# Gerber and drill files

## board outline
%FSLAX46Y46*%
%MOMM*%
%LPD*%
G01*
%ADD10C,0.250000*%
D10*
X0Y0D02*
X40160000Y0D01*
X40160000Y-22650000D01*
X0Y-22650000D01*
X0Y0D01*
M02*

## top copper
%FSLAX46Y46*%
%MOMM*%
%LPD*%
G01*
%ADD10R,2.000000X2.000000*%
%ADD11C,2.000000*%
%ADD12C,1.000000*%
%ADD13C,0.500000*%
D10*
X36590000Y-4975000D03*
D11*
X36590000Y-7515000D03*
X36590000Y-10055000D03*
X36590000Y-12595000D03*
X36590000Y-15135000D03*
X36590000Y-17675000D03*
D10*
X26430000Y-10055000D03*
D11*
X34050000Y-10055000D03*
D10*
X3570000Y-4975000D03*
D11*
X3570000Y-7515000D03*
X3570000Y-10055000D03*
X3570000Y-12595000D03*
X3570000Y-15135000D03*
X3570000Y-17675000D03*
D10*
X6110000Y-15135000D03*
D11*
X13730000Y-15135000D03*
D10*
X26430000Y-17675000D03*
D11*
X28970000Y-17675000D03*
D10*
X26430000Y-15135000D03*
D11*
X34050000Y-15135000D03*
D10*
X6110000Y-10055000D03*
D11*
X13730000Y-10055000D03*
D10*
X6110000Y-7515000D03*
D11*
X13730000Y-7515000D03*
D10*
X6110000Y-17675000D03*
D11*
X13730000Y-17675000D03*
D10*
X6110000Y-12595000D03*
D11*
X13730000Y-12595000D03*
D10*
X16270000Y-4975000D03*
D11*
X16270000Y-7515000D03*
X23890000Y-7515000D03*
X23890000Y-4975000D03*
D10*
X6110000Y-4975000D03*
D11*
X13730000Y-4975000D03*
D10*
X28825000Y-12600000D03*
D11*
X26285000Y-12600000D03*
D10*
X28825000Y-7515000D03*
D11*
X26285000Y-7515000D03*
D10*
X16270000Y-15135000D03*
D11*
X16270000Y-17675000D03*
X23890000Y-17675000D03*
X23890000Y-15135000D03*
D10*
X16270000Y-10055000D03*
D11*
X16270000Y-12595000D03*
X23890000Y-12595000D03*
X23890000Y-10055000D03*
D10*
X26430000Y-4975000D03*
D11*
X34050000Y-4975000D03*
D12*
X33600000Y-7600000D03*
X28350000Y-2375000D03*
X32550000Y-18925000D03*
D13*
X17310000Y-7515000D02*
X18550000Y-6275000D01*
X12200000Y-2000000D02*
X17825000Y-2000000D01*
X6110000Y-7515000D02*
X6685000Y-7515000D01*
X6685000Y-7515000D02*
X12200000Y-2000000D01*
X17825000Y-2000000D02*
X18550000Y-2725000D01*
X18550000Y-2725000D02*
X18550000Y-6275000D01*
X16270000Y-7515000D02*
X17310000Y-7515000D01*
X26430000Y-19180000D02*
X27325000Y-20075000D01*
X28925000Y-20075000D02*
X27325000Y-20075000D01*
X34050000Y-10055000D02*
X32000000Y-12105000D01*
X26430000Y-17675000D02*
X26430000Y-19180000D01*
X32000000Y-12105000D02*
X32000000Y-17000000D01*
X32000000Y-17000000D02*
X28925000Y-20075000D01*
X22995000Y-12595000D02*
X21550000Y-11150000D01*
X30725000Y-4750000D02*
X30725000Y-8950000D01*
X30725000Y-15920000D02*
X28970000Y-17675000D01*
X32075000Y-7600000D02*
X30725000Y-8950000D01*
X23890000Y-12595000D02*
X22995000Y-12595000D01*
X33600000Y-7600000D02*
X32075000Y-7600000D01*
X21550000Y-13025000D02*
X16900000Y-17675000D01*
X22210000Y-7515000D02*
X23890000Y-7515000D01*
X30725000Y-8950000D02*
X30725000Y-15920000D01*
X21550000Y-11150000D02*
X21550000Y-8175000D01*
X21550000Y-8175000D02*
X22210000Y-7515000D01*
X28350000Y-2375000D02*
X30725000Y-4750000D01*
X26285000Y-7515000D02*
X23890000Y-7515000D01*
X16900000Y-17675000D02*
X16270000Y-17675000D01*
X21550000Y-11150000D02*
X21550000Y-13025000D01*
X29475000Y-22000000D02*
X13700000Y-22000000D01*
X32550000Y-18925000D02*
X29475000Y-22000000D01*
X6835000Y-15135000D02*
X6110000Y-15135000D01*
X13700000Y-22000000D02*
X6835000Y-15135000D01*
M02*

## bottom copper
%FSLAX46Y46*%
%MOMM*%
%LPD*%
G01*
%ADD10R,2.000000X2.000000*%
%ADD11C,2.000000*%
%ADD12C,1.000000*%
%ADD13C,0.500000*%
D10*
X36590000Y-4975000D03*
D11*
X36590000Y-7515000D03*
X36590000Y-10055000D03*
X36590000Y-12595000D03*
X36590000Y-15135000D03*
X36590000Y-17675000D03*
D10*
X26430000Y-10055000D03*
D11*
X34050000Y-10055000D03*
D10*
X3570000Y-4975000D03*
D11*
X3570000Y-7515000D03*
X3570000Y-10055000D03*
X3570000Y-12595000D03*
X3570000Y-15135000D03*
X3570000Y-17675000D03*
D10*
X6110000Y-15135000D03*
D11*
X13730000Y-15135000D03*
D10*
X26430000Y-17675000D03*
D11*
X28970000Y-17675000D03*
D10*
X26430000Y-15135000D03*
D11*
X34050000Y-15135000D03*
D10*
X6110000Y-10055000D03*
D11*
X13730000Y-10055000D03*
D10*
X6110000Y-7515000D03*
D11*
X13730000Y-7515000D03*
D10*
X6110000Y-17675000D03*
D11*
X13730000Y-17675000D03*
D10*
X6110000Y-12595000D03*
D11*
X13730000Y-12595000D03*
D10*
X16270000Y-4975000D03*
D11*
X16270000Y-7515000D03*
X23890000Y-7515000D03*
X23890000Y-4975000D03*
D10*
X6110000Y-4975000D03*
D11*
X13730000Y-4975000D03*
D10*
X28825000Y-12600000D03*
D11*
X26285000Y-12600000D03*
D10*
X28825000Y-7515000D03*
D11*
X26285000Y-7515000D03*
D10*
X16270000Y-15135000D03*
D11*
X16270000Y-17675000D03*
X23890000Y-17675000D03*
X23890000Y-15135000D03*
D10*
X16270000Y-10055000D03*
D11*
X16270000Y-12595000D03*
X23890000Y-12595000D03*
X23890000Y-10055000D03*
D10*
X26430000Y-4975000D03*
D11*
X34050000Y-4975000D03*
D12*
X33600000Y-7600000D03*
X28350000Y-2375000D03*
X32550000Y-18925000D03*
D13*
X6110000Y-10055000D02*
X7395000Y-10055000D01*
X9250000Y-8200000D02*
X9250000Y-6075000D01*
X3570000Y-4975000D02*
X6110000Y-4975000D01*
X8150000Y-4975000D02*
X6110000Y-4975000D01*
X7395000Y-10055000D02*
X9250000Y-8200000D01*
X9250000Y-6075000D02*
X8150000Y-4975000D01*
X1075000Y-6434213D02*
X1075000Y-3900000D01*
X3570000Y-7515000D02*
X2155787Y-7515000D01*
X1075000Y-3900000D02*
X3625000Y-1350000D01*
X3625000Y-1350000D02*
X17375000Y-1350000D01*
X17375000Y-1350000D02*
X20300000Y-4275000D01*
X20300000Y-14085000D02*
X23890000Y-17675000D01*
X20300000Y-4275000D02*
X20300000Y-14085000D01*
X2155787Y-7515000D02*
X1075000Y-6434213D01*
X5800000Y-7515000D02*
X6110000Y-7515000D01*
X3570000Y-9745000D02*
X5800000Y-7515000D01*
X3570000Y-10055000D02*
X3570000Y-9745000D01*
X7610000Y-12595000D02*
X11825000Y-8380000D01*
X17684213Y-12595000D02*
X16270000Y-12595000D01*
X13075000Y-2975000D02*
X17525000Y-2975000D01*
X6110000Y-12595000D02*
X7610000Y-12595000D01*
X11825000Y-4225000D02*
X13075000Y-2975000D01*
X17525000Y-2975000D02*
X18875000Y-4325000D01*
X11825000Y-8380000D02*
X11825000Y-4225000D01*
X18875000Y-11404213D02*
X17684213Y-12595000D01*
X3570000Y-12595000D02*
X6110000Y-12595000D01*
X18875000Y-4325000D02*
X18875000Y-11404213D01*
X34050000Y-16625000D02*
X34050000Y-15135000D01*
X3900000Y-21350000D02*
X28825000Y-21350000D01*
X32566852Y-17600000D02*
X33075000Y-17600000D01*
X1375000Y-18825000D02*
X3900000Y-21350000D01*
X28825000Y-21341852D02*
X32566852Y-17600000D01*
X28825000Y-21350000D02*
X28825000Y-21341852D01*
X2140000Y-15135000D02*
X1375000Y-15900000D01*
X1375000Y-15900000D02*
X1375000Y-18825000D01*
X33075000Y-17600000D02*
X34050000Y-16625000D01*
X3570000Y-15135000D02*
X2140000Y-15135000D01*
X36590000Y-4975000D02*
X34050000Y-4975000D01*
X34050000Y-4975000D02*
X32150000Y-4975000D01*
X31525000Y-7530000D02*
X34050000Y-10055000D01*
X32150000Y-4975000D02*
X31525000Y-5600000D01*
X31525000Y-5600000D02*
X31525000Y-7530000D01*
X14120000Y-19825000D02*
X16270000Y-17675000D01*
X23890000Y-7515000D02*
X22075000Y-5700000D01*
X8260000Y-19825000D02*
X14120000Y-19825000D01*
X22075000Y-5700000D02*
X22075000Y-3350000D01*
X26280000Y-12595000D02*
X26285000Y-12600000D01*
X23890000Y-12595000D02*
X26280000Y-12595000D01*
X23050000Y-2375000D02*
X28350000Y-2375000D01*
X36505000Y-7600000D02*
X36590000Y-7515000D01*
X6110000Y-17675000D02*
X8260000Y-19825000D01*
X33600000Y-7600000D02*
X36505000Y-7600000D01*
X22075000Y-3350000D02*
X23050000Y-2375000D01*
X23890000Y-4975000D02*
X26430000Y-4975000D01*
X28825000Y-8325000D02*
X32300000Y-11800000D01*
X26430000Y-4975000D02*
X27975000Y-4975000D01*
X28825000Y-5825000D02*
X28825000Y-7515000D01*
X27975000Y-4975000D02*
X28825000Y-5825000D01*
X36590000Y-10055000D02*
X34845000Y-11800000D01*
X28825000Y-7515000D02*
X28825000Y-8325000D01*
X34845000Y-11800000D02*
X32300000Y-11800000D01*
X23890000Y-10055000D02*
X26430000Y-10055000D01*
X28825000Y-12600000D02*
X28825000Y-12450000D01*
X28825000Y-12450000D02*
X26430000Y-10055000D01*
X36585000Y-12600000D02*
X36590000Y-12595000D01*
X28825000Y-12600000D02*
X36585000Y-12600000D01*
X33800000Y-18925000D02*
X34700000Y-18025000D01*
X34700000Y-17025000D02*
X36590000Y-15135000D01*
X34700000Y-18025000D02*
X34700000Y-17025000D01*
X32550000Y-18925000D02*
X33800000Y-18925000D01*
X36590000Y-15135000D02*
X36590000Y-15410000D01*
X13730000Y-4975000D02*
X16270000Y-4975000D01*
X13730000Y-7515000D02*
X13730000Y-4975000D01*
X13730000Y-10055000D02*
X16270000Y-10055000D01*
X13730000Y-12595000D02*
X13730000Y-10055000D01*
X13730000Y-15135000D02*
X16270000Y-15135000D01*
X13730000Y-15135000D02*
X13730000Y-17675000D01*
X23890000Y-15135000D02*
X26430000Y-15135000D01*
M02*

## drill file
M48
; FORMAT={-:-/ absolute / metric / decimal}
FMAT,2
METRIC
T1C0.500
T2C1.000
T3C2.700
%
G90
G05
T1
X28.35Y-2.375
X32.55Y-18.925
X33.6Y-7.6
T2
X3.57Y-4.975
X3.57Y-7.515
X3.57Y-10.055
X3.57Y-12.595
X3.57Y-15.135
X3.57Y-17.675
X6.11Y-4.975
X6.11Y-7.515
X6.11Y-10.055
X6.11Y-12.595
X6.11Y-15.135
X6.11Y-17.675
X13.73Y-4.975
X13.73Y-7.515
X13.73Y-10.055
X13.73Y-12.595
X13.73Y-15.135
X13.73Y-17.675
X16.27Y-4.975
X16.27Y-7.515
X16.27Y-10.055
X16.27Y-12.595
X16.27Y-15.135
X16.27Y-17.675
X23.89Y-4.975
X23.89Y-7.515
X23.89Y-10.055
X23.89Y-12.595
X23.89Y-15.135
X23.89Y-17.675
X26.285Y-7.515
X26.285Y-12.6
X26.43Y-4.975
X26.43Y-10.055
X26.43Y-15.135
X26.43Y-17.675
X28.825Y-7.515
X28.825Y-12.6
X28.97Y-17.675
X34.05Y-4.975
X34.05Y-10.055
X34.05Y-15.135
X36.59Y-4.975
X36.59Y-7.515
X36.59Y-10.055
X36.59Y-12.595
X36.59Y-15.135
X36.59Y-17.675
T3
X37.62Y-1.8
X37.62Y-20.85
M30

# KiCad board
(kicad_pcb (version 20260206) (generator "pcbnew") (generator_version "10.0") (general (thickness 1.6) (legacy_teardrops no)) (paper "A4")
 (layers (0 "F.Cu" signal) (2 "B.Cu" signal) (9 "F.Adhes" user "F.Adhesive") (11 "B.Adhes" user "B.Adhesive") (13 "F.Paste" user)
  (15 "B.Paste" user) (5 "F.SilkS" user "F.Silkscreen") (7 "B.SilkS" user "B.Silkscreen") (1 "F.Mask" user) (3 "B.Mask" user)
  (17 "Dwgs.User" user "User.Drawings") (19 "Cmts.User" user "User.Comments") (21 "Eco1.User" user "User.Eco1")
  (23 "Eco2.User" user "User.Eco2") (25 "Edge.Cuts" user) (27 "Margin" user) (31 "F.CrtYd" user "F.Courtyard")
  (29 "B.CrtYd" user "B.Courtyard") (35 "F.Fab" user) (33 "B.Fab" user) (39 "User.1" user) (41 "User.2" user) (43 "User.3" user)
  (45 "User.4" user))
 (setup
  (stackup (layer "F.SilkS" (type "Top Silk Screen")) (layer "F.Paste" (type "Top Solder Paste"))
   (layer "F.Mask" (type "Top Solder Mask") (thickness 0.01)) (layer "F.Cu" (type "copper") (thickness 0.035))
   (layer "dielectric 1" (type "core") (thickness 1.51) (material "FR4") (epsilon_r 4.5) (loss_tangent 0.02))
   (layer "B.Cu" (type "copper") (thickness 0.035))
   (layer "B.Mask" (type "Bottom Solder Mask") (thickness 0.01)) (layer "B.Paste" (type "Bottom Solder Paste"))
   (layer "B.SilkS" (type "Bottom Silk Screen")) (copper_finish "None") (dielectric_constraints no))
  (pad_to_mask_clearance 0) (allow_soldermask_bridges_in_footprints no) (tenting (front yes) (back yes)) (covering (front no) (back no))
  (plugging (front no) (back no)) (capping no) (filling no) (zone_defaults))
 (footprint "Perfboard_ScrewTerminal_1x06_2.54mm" (layer "F.Cu") (at 36.59 4.975)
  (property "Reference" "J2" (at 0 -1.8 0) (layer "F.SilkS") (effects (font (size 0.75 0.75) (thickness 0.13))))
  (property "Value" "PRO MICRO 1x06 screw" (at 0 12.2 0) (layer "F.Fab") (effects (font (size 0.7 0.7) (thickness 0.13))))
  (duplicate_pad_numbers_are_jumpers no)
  (pad "1" thru_hole rect (at 0 0) (size 2 2) (drill 1) (layers "*.Cu" "*.Mask") (remove_unused_layers no) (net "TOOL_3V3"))
  (pad "2" thru_hole circle (at 0 2.54) (size 2 2) (drill 1) (layers "*.Cu" "*.Mask") (remove_unused_layers no) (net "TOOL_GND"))
  (pad "3" thru_hole circle (at 0 5.08) (size 2 2) (drill 1) (layers "*.Cu" "*.Mask") (remove_unused_layers no) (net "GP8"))
  (pad "4" thru_hole circle (at 0 7.62) (size 2 2) (drill 1) (layers "*.Cu" "*.Mask") (remove_unused_layers no) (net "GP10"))
  (pad "5" thru_hole circle (at 0 10.16) (size 2 2) (drill 1) (layers "*.Cu" "*.Mask") (remove_unused_layers no) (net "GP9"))
  (pad "6" thru_hole circle (at 0 12.7) (size 2 2) (drill 1) (layers "*.Cu" "*.Mask") (remove_unused_layers no)))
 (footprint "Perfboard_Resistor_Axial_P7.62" (layer "F.Cu") (at 26.43 10.055)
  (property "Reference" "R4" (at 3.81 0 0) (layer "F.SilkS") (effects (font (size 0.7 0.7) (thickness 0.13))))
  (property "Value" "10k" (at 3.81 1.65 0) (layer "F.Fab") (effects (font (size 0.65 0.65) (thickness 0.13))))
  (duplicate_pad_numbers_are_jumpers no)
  (pad "1" thru_hole rect (at 0 0) (size 2 2) (drill 1) (layers "*.Cu" "*.Mask") (remove_unused_layers no) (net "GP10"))
  (pad "2" thru_hole circle (at 7.62 0) (size 2 2) (drill 1) (layers "*.Cu" "*.Mask") (remove_unused_layers no) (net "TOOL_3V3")))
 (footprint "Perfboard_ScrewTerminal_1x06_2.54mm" (layer "F.Cu") (at 3.57 4.975)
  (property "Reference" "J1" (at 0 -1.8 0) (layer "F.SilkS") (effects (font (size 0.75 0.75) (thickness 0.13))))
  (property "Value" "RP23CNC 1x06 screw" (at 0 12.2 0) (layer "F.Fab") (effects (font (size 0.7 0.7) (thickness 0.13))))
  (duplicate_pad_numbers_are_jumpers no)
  (pad "1" thru_hole rect (at 0 0) (size 2 2) (drill 1) (layers "*.Cu" "*.Mask") (remove_unused_layers no) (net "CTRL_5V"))
  (pad "2" thru_hole circle (at 0 2.54) (size 2 2) (drill 1) (layers "*.Cu" "*.Mask") (remove_unused_layers no) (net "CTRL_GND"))
  (pad "3" thru_hole circle (at 0 5.08) (size 2 2) (drill 1) (layers "*.Cu" "*.Mask") (remove_unused_layers no) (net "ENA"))
  (pad "4" thru_hole circle (at 0 7.62) (size 2 2) (drill 1) (layers "*.Cu" "*.Mask") (remove_unused_layers no) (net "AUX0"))
  (pad "5" thru_hole circle (at 0 10.16) (size 2 2) (drill 1) (layers "*.Cu" "*.Mask") (remove_unused_layers no) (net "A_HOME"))
  (pad "6" thru_hole circle (at 0 12.7) (size 2 2) (drill 1) (layers "*.Cu" "*.Mask") (remove_unused_layers no)))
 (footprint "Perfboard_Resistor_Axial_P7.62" (layer "F.Cu") (at 6.11 15.135)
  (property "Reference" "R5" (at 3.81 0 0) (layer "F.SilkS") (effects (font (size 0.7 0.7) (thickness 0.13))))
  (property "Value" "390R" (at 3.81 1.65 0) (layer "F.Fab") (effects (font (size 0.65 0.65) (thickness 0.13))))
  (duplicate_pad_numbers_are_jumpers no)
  (pad "1" thru_hole rect (at 0 0) (size 2 2) (drill 1) (layers "*.Cu" "*.Mask") (remove_unused_layers no) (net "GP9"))
  (pad "2" thru_hole circle (at 7.62 0) (size 2 2) (drill 1) (layers "*.Cu" "*.Mask") (remove_unused_layers no) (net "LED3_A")))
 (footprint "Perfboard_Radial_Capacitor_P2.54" (layer "F.Cu") (at 26.43 17.675)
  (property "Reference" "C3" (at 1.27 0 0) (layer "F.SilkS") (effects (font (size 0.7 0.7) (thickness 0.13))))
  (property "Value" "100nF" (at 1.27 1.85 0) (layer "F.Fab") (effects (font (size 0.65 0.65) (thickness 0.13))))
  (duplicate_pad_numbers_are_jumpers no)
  (pad "1" thru_hole rect (at 0 0) (size 2 2) (drill 1) (layers "*.Cu" "*.Mask") (remove_unused_layers no) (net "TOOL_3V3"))
  (pad "2" thru_hole circle (at 2.54 0) (size 2 2) (drill 1) (layers "*.Cu" "*.Mask") (remove_unused_layers no) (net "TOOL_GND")))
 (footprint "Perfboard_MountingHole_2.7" (layer "F.Cu") (at 37.62 1.8)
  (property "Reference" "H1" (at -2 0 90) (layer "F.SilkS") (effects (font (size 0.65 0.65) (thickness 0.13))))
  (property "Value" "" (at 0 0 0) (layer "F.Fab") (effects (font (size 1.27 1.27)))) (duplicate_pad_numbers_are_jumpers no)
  (pad "" np_thru_hole circle (at 0 0) (size 2.7 2.7) (drill 2.7) (layers "*.Cu" "*.Mask")))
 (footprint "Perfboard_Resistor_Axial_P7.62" (layer "F.Cu") (at 26.43 15.135)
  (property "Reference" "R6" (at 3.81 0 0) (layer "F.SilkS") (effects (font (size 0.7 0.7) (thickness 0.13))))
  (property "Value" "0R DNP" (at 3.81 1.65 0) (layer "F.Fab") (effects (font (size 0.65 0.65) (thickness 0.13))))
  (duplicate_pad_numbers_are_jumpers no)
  (pad "1" thru_hole rect (at 0 0) (size 2 2) (drill 1) (layers "*.Cu" "*.Mask") (remove_unused_layers no) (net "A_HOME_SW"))
  (pad "2" thru_hole circle (at 7.62 0) (size 2 2) (drill 1) (layers "*.Cu" "*.Mask") (remove_unused_layers no) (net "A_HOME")))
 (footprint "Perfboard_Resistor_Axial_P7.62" (layer "F.Cu") (at 6.11 10.055)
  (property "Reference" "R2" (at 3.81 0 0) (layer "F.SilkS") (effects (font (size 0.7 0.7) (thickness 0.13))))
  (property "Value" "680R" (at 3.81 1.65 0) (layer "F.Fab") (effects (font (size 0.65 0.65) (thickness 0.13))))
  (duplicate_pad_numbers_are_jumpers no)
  (pad "1" thru_hole rect (at 0 0) (size 2 2) (drill 1) (layers "*.Cu" "*.Mask") (remove_unused_layers no) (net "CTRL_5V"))
  (pad "2" thru_hole circle (at 7.62 0) (size 2 2) (drill 1) (layers "*.Cu" "*.Mask") (remove_unused_layers no) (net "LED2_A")))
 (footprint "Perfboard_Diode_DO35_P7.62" (layer "F.Cu") (at 6.11 7.515)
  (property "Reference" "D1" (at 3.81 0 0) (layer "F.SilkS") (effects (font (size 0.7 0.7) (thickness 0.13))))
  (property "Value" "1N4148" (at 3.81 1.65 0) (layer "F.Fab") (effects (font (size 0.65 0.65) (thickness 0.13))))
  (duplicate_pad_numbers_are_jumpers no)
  (pad "1" thru_hole rect (at 0 0) (size 2 2) (drill 1) (layers "*.Cu" "*.Mask") (remove_unused_layers no) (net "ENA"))
  (pad "2" thru_hole circle (at 7.62 0) (size 2 2) (drill 1) (layers "*.Cu" "*.Mask") (remove_unused_layers no) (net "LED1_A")))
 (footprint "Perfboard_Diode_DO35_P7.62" (layer "F.Cu") (at 6.11 17.675)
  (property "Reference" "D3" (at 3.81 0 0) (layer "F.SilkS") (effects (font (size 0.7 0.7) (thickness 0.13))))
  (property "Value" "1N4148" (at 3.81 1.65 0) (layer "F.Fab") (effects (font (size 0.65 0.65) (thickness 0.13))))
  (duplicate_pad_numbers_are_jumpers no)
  (pad "1" thru_hole rect (at 0 0) (size 2 2) (drill 1) (layers "*.Cu" "*.Mask") (remove_unused_layers no) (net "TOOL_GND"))
  (pad "2" thru_hole circle (at 7.62 0) (size 2 2) (drill 1) (layers "*.Cu" "*.Mask") (remove_unused_layers no) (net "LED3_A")))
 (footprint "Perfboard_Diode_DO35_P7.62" (layer "F.Cu") (at 6.11 12.595)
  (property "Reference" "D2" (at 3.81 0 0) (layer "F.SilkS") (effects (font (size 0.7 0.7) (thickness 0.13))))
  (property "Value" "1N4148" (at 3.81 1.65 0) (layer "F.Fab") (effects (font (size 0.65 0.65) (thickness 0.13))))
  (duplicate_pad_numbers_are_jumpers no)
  (pad "1" thru_hole rect (at 0 0) (size 2 2) (drill 1) (layers "*.Cu" "*.Mask") (remove_unused_layers no) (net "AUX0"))
  (pad "2" thru_hole circle (at 7.62 0) (size 2 2) (drill 1) (layers "*.Cu" "*.Mask") (remove_unused_layers no) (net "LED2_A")))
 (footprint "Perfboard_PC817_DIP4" (layer "F.Cu") (at 16.27 4.975)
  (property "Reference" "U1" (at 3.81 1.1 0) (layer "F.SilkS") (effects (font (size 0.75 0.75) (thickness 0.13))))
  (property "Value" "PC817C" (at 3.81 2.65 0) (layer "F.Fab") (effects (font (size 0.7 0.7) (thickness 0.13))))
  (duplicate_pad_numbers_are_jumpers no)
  (pad "1" thru_hole rect (at 0 0) (size 2 2) (drill 1) (layers "*.Cu" "*.Mask") (remove_unused_layers no) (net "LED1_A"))
  (pad "2" thru_hole circle (at 0 2.54) (size 2 2) (drill 1) (layers "*.Cu" "*.Mask") (remove_unused_layers no) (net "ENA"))
  (pad "3" thru_hole circle (at 7.62 2.54) (size 2 2) (drill 1) (layers "*.Cu" "*.Mask") (remove_unused_layers no) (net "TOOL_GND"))
  (pad "4" thru_hole circle (at 7.62 0) (size 2 2) (drill 1) (layers "*.Cu" "*.Mask") (remove_unused_layers no) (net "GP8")))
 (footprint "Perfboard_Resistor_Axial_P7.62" (layer "F.Cu") (at 6.11 4.975)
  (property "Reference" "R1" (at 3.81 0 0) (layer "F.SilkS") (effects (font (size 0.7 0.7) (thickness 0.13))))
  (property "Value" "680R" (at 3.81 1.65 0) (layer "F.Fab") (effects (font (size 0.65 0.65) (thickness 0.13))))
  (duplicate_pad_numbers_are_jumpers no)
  (pad "1" thru_hole rect (at 0 0) (size 2 2) (drill 1) (layers "*.Cu" "*.Mask") (remove_unused_layers no) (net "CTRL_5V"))
  (pad "2" thru_hole circle (at 7.62 0) (size 2 2) (drill 1) (layers "*.Cu" "*.Mask") (remove_unused_layers no) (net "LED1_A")))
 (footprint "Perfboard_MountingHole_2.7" (layer "F.Cu") (at 37.62 20.85)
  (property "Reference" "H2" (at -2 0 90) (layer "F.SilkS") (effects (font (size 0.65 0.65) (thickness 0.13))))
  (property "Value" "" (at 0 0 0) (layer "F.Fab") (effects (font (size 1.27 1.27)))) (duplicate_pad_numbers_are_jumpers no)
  (pad "" np_thru_hole circle (at 0 0) (size 2.7 2.7) (drill 2.7) (layers "*.Cu" "*.Mask")))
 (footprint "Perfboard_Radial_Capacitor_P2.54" (layer "F.Cu") (at 28.825 12.6 180)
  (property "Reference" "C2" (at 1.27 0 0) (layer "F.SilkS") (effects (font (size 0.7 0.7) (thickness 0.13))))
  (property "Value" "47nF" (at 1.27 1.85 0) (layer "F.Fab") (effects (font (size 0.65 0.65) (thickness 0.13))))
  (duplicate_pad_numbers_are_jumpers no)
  (pad "1" thru_hole rect (at 0 0 180) (size 2 2) (drill 1) (layers "*.Cu" "*.Mask") (remove_unused_layers no) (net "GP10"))
  (pad "2" thru_hole circle (at 2.54 0 180) (size 2 2) (drill 1) (layers "*.Cu" "*.Mask") (remove_unused_layers no) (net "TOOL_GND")))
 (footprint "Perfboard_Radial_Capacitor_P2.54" (layer "F.Cu") (at 28.825 7.515 180)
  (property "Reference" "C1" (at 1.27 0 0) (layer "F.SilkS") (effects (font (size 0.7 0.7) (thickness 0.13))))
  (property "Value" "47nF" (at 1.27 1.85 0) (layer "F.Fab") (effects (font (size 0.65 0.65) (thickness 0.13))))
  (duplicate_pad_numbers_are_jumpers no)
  (pad "1" thru_hole rect (at 0 0 180) (size 2 2) (drill 1) (layers "*.Cu" "*.Mask") (remove_unused_layers no) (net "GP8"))
  (pad "2" thru_hole circle (at 2.54 0 180) (size 2 2) (drill 1) (layers "*.Cu" "*.Mask") (remove_unused_layers no) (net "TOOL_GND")))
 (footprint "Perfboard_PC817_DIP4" (layer "F.Cu") (at 16.27 15.135)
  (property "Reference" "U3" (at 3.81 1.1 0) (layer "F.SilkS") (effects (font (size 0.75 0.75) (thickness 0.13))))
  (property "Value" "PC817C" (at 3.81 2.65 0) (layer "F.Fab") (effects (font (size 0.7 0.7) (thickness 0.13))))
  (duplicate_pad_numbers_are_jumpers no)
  (pad "1" thru_hole rect (at 0 0) (size 2 2) (drill 1) (layers "*.Cu" "*.Mask") (remove_unused_layers no) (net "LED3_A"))
  (pad "2" thru_hole circle (at 0 2.54) (size 2 2) (drill 1) (layers "*.Cu" "*.Mask") (remove_unused_layers no) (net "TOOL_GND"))
  (pad "3" thru_hole circle (at 7.62 2.54) (size 2 2) (drill 1) (layers "*.Cu" "*.Mask") (remove_unused_layers no) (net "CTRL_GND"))
  (pad "4" thru_hole circle (at 7.62 0) (size 2 2) (drill 1) (layers "*.Cu" "*.Mask") (remove_unused_layers no) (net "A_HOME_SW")))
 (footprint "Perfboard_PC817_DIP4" (layer "F.Cu") (at 16.27 10.055)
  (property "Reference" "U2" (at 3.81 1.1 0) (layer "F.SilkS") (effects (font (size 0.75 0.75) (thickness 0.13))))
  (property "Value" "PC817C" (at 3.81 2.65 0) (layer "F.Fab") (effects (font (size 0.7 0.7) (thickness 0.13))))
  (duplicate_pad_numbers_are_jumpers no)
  (pad "1" thru_hole rect (at 0 0) (size 2 2) (drill 1) (layers "*.Cu" "*.Mask") (remove_unused_layers no) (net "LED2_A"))
  (pad "2" thru_hole circle (at 0 2.54) (size 2 2) (drill 1) (layers "*.Cu" "*.Mask") (remove_unused_layers no) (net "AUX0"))
  (pad "3" thru_hole circle (at 7.62 2.54) (size 2 2) (drill 1) (layers "*.Cu" "*.Mask") (remove_unused_layers no) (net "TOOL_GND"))
  (pad "4" thru_hole circle (at 7.62 0) (size 2 2) (drill 1) (layers "*.Cu" "*.Mask") (remove_unused_layers no) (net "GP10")))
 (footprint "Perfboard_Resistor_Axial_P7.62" (layer "F.Cu") (at 26.43 4.975)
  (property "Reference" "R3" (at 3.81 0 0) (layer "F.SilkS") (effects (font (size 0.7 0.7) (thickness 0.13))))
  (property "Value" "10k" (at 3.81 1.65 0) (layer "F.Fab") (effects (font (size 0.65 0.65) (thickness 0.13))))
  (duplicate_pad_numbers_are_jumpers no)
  (pad "1" thru_hole rect (at 0 0) (size 2 2) (drill 1) (layers "*.Cu" "*.Mask") (remove_unused_layers no) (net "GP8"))
  (pad "2" thru_hole circle (at 7.62 0) (size 2 2) (drill 1) (layers "*.Cu" "*.Mask") (remove_unused_layers no) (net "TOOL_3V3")))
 (gr_rect (start 0 0) (end 40.16 22.65) (stroke (width 0.25) (type default)) (fill no) (layer "Edge.Cuts"))
 (segment (start 6.11 10.055) (end 7.395 10.055) (width 0.5) (layer "B.Cu") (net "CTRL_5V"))
 (segment (start 9.25 8.2) (end 9.25 6.075) (width 0.5) (layer "B.Cu") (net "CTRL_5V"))
 (segment (start 3.57 4.975) (end 6.11 4.975) (width 0.5) (layer "B.Cu") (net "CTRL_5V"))
 (segment (start 8.15 4.975) (end 6.11 4.975) (width 0.5) (layer "B.Cu") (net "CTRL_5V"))
 (segment (start 7.395 10.055) (end 9.25 8.2) (width 0.5) (layer "B.Cu") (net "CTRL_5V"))
 (segment (start 9.25 6.075) (end 8.15 4.975) (width 0.5) (layer "B.Cu") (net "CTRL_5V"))
 (segment (start 1.075 6.434213) (end 1.075 3.9) (width 0.5) (layer "B.Cu") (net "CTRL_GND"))
 (segment (start 3.57 7.515) (end 2.155787 7.515) (width 0.5) (layer "B.Cu") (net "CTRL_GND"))
 (segment (start 1.075 3.9) (end 3.625 1.35) (width 0.5) (layer "B.Cu") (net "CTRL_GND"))
 (segment (start 3.625 1.35) (end 17.375 1.35) (width 0.5) (layer "B.Cu") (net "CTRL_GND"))
 (segment (start 17.375 1.35) (end 20.3 4.275) (width 0.5) (layer "B.Cu") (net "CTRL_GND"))
 (segment (start 20.3 14.085) (end 23.89 17.675) (width 0.5) (layer "B.Cu") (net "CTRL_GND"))
 (segment (start 20.3 4.275) (end 20.3 14.085) (width 0.5) (layer "B.Cu") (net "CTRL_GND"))
 (segment (start 2.155787 7.515) (end 1.075 6.434213) (width 0.5) (layer "B.Cu") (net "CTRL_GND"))
 (segment (start 17.31 7.515) (end 18.55 6.275) (width 0.5) (layer "F.Cu") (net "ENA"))
 (segment (start 12.2 2) (end 17.825 2) (width 0.5) (layer "F.Cu") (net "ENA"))
 (segment (start 6.11 7.515) (end 6.685 7.515) (width 0.5) (layer "F.Cu") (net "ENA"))
 (segment (start 6.685 7.515) (end 12.2 2) (width 0.5) (layer "F.Cu") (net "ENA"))
 (segment (start 17.825 2) (end 18.55 2.725) (width 0.5) (layer "F.Cu") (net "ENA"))
 (segment (start 18.55 2.725) (end 18.55 6.275) (width 0.5) (layer "F.Cu") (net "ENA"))
 (segment (start 16.27 7.515) (end 17.31 7.515) (width 0.5) (layer "F.Cu") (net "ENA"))
 (segment (start 5.8 7.515) (end 6.11 7.515) (width 0.5) (layer "B.Cu") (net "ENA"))
 (segment (start 3.57 9.745) (end 5.8 7.515) (width 0.5) (layer "B.Cu") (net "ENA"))
 (segment (start 3.57 10.055) (end 3.57 9.745) (width 0.5) (layer "B.Cu") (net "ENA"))
 (segment (start 7.61 12.595) (end 11.825 8.38) (width 0.5) (layer "B.Cu") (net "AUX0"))
 (segment (start 17.684213 12.595) (end 16.27 12.595) (width 0.5) (layer "B.Cu") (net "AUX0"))
 (segment (start 13.075 2.975) (end 17.525 2.975) (width 0.5) (layer "B.Cu") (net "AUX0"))
 (segment (start 6.11 12.595) (end 7.61 12.595) (width 0.5) (layer "B.Cu") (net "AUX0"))
 (segment (start 11.825 4.225) (end 13.075 2.975) (width 0.5) (layer "B.Cu") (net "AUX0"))
 (segment (start 17.525 2.975) (end 18.875 4.325) (width 0.5) (layer "B.Cu") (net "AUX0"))
 (segment (start 11.825 8.38) (end 11.825 4.225) (width 0.5) (layer "B.Cu") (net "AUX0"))
 (segment (start 18.875 11.404213) (end 17.684213 12.595) (width 0.5) (layer "B.Cu") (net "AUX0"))
 (segment (start 3.57 12.595) (end 6.11 12.595) (width 0.5) (layer "B.Cu") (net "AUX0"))
 (segment (start 18.875 4.325) (end 18.875 11.404213) (width 0.5) (layer "B.Cu") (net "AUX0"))
 (segment (start 34.05 16.625) (end 34.05 15.135) (width 0.5) (layer "B.Cu") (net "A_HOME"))
 (segment (start 3.9 21.35) (end 28.825 21.35) (width 0.5) (layer "B.Cu") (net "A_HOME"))
 (segment (start 32.566852 17.6) (end 33.075 17.6) (width 0.5) (layer "B.Cu") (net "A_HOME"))
 (segment (start 1.375 18.825) (end 3.9 21.35) (width 0.5) (layer "B.Cu") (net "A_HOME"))
 (segment (start 28.825 21.341852) (end 32.566852 17.6) (width 0.5) (layer "B.Cu") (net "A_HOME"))
 (segment (start 28.825 21.35) (end 28.825 21.341852) (width 0.5) (layer "B.Cu") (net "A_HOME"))
 (segment (start 2.14 15.135) (end 1.375 15.9) (width 0.5) (layer "B.Cu") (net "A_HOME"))
 (segment (start 1.375 15.9) (end 1.375 18.825) (width 0.5) (layer "B.Cu") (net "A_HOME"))
 (segment (start 33.075 17.6) (end 34.05 16.625) (width 0.5) (layer "B.Cu") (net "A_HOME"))
 (segment (start 3.57 15.135) (end 2.14 15.135) (width 0.5) (layer "B.Cu") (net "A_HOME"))
 (segment (start 26.43 19.18) (end 27.325 20.075) (width 0.5) (layer "F.Cu") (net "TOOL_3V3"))
 (segment (start 28.925 20.075) (end 27.325 20.075) (width 0.5) (layer "F.Cu") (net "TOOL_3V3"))
 (segment (start 34.05 10.055) (end 32 12.105) (width 0.5) (layer "F.Cu") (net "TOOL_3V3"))
 (segment (start 26.43 17.675) (end 26.43 19.18) (width 0.5) (layer "F.Cu") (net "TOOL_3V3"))
 (segment (start 32 12.105) (end 32 17) (width 0.5) (layer "F.Cu") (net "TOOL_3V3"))
 (segment (start 32 17) (end 28.925 20.075) (width 0.5) (layer "F.Cu") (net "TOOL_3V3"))
 (segment (start 36.59 4.975) (end 34.05 4.975) (width 0.5) (layer "B.Cu") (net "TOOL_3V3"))
 (segment (start 34.05 4.975) (end 32.15 4.975) (width 0.5) (layer "B.Cu") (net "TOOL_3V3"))
 (segment (start 31.525 7.53) (end 34.05 10.055) (width 0.5) (layer "B.Cu") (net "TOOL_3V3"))
 (segment (start 32.15 4.975) (end 31.525 5.6) (width 0.5) (layer "B.Cu") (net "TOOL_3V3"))
 (segment (start 31.525 5.6) (end 31.525 7.53) (width 0.5) (layer "B.Cu") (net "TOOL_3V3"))
 (segment (start 22.995 12.595) (end 21.55 11.15) (width 0.5) (layer "F.Cu") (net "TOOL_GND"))
 (segment (start 30.725 4.75) (end 30.725 8.95) (width 0.5) (layer "F.Cu") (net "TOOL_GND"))
 (segment (start 30.725 15.92) (end 28.97 17.675) (width 0.5) (layer "F.Cu") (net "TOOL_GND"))
 (segment (start 32.075 7.6) (end 30.725 8.95) (width 0.5) (layer "F.Cu") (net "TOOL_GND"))
 (segment (start 23.89 12.595) (end 22.995 12.595) (width 0.5) (layer "F.Cu") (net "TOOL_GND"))
 (segment (start 33.6 7.6) (end 32.075 7.6) (width 0.5) (layer "F.Cu") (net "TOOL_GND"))
 (segment (start 21.55 13.025) (end 16.9 17.675) (width 0.5) (layer "F.Cu") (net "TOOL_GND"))
 (segment (start 22.21 7.515) (end 23.89 7.515) (width 0.5) (layer "F.Cu") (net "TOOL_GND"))
 (segment (start 30.725 8.95) (end 30.725 15.92) (width 0.5) (layer "F.Cu") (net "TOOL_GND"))
 (segment (start 21.55 11.15) (end 21.55 8.175) (width 0.5) (layer "F.Cu") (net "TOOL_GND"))
 (segment (start 21.55 8.175) (end 22.21 7.515) (width 0.5) (layer "F.Cu") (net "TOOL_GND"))
 (segment (start 28.35 2.375) (end 30.725 4.75) (width 0.5) (layer "F.Cu") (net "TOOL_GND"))
 (segment (start 26.285 7.515) (end 23.89 7.515) (width 0.5) (layer "F.Cu") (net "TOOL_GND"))
 (segment (start 16.9 17.675) (end 16.27 17.675) (width 0.5) (layer "F.Cu") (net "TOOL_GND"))
 (segment (start 21.55 11.15) (end 21.55 13.025) (width 0.5) (layer "F.Cu") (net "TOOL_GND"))
 (via (at 33.6 7.6) (size 1) (drill 0.5) (layers "F.Cu" "B.Cu") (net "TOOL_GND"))
 (via (at 28.35 2.375) (size 1) (drill 0.5) (layers "F.Cu" "B.Cu") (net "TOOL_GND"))
 (segment (start 14.12 19.825) (end 16.27 17.675) (width 0.5) (layer "B.Cu") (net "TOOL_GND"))
 (segment (start 23.89 7.515) (end 22.075 5.7) (width 0.5) (layer "B.Cu") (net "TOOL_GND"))
 (segment (start 8.26 19.825) (end 14.12 19.825) (width 0.5) (layer "B.Cu") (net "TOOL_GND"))
 (segment (start 22.075 5.7) (end 22.075 3.35) (width 0.5) (layer "B.Cu") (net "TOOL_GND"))
 (segment (start 26.28 12.595) (end 26.285 12.6) (width 0.5) (layer "B.Cu") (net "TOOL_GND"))
 (segment (start 23.89 12.595) (end 26.28 12.595) (width 0.5) (layer "B.Cu") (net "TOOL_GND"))
 (segment (start 23.05 2.375) (end 28.35 2.375) (width 0.5) (layer "B.Cu") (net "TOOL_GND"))
 (segment (start 36.505 7.6) (end 36.59 7.515) (width 0.5) (layer "B.Cu") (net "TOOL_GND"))
 (segment (start 6.11 17.675) (end 8.26 19.825) (width 0.5) (layer "B.Cu") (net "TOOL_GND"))
 (segment (start 33.6 7.6) (end 36.505 7.6) (width 0.5) (layer "B.Cu") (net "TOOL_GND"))
 (segment (start 22.075 3.35) (end 23.05 2.375) (width 0.5) (layer "B.Cu") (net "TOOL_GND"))
 (segment (start 23.89 4.975) (end 26.43 4.975) (width 0.5) (layer "B.Cu") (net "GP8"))
 (segment (start 28.825 8.325) (end 32.3 11.8) (width 0.5) (layer "B.Cu") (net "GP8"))
 (segment (start 26.43 4.975) (end 27.975 4.975) (width 0.5) (layer "B.Cu") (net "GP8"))
 (segment (start 28.825 5.825) (end 28.825 7.515) (width 0.5) (layer "B.Cu") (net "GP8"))
 (segment (start 27.975 4.975) (end 28.825 5.825) (width 0.5) (layer "B.Cu") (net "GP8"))
 (segment (start 36.59 10.055) (end 34.845 11.8) (width 0.5) (layer "B.Cu") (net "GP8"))
 (segment (start 28.825 7.515) (end 28.825 8.325) (width 0.5) (layer "B.Cu") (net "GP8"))
 (segment (start 34.845 11.8) (end 32.3 11.8) (width 0.5) (layer "B.Cu") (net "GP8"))
 (segment (start 23.89 10.055) (end 26.43 10.055) (width 0.5) (layer "B.Cu") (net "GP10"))
 (segment (start 28.825 12.6) (end 28.825 12.45) (width 0.5) (layer "B.Cu") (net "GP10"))
 (segment (start 28.825 12.45) (end 26.43 10.055) (width 0.5) (layer "B.Cu") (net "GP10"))
 (segment (start 36.585 12.6) (end 36.59 12.595) (width 0.5) (layer "B.Cu") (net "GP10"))
 (segment (start 28.825 12.6) (end 36.585 12.6) (width 0.5) (layer "B.Cu") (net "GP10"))
 (segment (start 29.475 22) (end 13.7 22) (width 0.5) (layer "F.Cu") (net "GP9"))
 (segment (start 32.55 18.925) (end 29.475 22) (width 0.5) (layer "F.Cu") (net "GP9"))
 (segment (start 6.835 15.135) (end 6.11 15.135) (width 0.5) (layer "F.Cu") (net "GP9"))
 (segment (start 13.7 22) (end 6.835 15.135) (width 0.5) (layer "F.Cu") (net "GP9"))
 (via (at 32.55 18.925) (size 1) (drill 0.5) (layers "F.Cu" "B.Cu") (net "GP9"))
 (segment (start 33.8 18.925) (end 34.7 18.025) (width 0.5) (layer "B.Cu") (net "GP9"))
 (segment (start 34.7 17.025) (end 36.59 15.135) (width 0.5) (layer "B.Cu") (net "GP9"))
 (segment (start 34.7 18.025) (end 34.7 17.025) (width 0.5) (layer "B.Cu") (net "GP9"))
 (segment (start 32.55 18.925) (end 33.8 18.925) (width 0.5) (layer "B.Cu") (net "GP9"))
 (segment (start 36.59 15.135) (end 36.59 15.41) (width 0.5) (layer "B.Cu") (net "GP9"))
 (segment (start 13.73 4.975) (end 16.27 4.975) (width 0.5) (layer "B.Cu") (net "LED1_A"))
 (segment (start 13.73 7.515) (end 13.73 4.975) (width 0.5) (layer "B.Cu") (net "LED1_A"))
 (segment (start 13.73 10.055) (end 16.27 10.055) (width 0.5) (layer "B.Cu") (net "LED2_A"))
 (segment (start 13.73 12.595) (end 13.73 10.055) (width 0.5) (layer "B.Cu") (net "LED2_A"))
 (segment (start 13.73 15.135) (end 16.27 15.135) (width 0.5) (layer "B.Cu") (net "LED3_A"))
 (segment (start 13.73 15.135) (end 13.73 17.675) (width 0.5) (layer "B.Cu") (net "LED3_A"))
 (segment (start 23.89 15.135) (end 26.43 15.135) (width 0.5) (layer "B.Cu") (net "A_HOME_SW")))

